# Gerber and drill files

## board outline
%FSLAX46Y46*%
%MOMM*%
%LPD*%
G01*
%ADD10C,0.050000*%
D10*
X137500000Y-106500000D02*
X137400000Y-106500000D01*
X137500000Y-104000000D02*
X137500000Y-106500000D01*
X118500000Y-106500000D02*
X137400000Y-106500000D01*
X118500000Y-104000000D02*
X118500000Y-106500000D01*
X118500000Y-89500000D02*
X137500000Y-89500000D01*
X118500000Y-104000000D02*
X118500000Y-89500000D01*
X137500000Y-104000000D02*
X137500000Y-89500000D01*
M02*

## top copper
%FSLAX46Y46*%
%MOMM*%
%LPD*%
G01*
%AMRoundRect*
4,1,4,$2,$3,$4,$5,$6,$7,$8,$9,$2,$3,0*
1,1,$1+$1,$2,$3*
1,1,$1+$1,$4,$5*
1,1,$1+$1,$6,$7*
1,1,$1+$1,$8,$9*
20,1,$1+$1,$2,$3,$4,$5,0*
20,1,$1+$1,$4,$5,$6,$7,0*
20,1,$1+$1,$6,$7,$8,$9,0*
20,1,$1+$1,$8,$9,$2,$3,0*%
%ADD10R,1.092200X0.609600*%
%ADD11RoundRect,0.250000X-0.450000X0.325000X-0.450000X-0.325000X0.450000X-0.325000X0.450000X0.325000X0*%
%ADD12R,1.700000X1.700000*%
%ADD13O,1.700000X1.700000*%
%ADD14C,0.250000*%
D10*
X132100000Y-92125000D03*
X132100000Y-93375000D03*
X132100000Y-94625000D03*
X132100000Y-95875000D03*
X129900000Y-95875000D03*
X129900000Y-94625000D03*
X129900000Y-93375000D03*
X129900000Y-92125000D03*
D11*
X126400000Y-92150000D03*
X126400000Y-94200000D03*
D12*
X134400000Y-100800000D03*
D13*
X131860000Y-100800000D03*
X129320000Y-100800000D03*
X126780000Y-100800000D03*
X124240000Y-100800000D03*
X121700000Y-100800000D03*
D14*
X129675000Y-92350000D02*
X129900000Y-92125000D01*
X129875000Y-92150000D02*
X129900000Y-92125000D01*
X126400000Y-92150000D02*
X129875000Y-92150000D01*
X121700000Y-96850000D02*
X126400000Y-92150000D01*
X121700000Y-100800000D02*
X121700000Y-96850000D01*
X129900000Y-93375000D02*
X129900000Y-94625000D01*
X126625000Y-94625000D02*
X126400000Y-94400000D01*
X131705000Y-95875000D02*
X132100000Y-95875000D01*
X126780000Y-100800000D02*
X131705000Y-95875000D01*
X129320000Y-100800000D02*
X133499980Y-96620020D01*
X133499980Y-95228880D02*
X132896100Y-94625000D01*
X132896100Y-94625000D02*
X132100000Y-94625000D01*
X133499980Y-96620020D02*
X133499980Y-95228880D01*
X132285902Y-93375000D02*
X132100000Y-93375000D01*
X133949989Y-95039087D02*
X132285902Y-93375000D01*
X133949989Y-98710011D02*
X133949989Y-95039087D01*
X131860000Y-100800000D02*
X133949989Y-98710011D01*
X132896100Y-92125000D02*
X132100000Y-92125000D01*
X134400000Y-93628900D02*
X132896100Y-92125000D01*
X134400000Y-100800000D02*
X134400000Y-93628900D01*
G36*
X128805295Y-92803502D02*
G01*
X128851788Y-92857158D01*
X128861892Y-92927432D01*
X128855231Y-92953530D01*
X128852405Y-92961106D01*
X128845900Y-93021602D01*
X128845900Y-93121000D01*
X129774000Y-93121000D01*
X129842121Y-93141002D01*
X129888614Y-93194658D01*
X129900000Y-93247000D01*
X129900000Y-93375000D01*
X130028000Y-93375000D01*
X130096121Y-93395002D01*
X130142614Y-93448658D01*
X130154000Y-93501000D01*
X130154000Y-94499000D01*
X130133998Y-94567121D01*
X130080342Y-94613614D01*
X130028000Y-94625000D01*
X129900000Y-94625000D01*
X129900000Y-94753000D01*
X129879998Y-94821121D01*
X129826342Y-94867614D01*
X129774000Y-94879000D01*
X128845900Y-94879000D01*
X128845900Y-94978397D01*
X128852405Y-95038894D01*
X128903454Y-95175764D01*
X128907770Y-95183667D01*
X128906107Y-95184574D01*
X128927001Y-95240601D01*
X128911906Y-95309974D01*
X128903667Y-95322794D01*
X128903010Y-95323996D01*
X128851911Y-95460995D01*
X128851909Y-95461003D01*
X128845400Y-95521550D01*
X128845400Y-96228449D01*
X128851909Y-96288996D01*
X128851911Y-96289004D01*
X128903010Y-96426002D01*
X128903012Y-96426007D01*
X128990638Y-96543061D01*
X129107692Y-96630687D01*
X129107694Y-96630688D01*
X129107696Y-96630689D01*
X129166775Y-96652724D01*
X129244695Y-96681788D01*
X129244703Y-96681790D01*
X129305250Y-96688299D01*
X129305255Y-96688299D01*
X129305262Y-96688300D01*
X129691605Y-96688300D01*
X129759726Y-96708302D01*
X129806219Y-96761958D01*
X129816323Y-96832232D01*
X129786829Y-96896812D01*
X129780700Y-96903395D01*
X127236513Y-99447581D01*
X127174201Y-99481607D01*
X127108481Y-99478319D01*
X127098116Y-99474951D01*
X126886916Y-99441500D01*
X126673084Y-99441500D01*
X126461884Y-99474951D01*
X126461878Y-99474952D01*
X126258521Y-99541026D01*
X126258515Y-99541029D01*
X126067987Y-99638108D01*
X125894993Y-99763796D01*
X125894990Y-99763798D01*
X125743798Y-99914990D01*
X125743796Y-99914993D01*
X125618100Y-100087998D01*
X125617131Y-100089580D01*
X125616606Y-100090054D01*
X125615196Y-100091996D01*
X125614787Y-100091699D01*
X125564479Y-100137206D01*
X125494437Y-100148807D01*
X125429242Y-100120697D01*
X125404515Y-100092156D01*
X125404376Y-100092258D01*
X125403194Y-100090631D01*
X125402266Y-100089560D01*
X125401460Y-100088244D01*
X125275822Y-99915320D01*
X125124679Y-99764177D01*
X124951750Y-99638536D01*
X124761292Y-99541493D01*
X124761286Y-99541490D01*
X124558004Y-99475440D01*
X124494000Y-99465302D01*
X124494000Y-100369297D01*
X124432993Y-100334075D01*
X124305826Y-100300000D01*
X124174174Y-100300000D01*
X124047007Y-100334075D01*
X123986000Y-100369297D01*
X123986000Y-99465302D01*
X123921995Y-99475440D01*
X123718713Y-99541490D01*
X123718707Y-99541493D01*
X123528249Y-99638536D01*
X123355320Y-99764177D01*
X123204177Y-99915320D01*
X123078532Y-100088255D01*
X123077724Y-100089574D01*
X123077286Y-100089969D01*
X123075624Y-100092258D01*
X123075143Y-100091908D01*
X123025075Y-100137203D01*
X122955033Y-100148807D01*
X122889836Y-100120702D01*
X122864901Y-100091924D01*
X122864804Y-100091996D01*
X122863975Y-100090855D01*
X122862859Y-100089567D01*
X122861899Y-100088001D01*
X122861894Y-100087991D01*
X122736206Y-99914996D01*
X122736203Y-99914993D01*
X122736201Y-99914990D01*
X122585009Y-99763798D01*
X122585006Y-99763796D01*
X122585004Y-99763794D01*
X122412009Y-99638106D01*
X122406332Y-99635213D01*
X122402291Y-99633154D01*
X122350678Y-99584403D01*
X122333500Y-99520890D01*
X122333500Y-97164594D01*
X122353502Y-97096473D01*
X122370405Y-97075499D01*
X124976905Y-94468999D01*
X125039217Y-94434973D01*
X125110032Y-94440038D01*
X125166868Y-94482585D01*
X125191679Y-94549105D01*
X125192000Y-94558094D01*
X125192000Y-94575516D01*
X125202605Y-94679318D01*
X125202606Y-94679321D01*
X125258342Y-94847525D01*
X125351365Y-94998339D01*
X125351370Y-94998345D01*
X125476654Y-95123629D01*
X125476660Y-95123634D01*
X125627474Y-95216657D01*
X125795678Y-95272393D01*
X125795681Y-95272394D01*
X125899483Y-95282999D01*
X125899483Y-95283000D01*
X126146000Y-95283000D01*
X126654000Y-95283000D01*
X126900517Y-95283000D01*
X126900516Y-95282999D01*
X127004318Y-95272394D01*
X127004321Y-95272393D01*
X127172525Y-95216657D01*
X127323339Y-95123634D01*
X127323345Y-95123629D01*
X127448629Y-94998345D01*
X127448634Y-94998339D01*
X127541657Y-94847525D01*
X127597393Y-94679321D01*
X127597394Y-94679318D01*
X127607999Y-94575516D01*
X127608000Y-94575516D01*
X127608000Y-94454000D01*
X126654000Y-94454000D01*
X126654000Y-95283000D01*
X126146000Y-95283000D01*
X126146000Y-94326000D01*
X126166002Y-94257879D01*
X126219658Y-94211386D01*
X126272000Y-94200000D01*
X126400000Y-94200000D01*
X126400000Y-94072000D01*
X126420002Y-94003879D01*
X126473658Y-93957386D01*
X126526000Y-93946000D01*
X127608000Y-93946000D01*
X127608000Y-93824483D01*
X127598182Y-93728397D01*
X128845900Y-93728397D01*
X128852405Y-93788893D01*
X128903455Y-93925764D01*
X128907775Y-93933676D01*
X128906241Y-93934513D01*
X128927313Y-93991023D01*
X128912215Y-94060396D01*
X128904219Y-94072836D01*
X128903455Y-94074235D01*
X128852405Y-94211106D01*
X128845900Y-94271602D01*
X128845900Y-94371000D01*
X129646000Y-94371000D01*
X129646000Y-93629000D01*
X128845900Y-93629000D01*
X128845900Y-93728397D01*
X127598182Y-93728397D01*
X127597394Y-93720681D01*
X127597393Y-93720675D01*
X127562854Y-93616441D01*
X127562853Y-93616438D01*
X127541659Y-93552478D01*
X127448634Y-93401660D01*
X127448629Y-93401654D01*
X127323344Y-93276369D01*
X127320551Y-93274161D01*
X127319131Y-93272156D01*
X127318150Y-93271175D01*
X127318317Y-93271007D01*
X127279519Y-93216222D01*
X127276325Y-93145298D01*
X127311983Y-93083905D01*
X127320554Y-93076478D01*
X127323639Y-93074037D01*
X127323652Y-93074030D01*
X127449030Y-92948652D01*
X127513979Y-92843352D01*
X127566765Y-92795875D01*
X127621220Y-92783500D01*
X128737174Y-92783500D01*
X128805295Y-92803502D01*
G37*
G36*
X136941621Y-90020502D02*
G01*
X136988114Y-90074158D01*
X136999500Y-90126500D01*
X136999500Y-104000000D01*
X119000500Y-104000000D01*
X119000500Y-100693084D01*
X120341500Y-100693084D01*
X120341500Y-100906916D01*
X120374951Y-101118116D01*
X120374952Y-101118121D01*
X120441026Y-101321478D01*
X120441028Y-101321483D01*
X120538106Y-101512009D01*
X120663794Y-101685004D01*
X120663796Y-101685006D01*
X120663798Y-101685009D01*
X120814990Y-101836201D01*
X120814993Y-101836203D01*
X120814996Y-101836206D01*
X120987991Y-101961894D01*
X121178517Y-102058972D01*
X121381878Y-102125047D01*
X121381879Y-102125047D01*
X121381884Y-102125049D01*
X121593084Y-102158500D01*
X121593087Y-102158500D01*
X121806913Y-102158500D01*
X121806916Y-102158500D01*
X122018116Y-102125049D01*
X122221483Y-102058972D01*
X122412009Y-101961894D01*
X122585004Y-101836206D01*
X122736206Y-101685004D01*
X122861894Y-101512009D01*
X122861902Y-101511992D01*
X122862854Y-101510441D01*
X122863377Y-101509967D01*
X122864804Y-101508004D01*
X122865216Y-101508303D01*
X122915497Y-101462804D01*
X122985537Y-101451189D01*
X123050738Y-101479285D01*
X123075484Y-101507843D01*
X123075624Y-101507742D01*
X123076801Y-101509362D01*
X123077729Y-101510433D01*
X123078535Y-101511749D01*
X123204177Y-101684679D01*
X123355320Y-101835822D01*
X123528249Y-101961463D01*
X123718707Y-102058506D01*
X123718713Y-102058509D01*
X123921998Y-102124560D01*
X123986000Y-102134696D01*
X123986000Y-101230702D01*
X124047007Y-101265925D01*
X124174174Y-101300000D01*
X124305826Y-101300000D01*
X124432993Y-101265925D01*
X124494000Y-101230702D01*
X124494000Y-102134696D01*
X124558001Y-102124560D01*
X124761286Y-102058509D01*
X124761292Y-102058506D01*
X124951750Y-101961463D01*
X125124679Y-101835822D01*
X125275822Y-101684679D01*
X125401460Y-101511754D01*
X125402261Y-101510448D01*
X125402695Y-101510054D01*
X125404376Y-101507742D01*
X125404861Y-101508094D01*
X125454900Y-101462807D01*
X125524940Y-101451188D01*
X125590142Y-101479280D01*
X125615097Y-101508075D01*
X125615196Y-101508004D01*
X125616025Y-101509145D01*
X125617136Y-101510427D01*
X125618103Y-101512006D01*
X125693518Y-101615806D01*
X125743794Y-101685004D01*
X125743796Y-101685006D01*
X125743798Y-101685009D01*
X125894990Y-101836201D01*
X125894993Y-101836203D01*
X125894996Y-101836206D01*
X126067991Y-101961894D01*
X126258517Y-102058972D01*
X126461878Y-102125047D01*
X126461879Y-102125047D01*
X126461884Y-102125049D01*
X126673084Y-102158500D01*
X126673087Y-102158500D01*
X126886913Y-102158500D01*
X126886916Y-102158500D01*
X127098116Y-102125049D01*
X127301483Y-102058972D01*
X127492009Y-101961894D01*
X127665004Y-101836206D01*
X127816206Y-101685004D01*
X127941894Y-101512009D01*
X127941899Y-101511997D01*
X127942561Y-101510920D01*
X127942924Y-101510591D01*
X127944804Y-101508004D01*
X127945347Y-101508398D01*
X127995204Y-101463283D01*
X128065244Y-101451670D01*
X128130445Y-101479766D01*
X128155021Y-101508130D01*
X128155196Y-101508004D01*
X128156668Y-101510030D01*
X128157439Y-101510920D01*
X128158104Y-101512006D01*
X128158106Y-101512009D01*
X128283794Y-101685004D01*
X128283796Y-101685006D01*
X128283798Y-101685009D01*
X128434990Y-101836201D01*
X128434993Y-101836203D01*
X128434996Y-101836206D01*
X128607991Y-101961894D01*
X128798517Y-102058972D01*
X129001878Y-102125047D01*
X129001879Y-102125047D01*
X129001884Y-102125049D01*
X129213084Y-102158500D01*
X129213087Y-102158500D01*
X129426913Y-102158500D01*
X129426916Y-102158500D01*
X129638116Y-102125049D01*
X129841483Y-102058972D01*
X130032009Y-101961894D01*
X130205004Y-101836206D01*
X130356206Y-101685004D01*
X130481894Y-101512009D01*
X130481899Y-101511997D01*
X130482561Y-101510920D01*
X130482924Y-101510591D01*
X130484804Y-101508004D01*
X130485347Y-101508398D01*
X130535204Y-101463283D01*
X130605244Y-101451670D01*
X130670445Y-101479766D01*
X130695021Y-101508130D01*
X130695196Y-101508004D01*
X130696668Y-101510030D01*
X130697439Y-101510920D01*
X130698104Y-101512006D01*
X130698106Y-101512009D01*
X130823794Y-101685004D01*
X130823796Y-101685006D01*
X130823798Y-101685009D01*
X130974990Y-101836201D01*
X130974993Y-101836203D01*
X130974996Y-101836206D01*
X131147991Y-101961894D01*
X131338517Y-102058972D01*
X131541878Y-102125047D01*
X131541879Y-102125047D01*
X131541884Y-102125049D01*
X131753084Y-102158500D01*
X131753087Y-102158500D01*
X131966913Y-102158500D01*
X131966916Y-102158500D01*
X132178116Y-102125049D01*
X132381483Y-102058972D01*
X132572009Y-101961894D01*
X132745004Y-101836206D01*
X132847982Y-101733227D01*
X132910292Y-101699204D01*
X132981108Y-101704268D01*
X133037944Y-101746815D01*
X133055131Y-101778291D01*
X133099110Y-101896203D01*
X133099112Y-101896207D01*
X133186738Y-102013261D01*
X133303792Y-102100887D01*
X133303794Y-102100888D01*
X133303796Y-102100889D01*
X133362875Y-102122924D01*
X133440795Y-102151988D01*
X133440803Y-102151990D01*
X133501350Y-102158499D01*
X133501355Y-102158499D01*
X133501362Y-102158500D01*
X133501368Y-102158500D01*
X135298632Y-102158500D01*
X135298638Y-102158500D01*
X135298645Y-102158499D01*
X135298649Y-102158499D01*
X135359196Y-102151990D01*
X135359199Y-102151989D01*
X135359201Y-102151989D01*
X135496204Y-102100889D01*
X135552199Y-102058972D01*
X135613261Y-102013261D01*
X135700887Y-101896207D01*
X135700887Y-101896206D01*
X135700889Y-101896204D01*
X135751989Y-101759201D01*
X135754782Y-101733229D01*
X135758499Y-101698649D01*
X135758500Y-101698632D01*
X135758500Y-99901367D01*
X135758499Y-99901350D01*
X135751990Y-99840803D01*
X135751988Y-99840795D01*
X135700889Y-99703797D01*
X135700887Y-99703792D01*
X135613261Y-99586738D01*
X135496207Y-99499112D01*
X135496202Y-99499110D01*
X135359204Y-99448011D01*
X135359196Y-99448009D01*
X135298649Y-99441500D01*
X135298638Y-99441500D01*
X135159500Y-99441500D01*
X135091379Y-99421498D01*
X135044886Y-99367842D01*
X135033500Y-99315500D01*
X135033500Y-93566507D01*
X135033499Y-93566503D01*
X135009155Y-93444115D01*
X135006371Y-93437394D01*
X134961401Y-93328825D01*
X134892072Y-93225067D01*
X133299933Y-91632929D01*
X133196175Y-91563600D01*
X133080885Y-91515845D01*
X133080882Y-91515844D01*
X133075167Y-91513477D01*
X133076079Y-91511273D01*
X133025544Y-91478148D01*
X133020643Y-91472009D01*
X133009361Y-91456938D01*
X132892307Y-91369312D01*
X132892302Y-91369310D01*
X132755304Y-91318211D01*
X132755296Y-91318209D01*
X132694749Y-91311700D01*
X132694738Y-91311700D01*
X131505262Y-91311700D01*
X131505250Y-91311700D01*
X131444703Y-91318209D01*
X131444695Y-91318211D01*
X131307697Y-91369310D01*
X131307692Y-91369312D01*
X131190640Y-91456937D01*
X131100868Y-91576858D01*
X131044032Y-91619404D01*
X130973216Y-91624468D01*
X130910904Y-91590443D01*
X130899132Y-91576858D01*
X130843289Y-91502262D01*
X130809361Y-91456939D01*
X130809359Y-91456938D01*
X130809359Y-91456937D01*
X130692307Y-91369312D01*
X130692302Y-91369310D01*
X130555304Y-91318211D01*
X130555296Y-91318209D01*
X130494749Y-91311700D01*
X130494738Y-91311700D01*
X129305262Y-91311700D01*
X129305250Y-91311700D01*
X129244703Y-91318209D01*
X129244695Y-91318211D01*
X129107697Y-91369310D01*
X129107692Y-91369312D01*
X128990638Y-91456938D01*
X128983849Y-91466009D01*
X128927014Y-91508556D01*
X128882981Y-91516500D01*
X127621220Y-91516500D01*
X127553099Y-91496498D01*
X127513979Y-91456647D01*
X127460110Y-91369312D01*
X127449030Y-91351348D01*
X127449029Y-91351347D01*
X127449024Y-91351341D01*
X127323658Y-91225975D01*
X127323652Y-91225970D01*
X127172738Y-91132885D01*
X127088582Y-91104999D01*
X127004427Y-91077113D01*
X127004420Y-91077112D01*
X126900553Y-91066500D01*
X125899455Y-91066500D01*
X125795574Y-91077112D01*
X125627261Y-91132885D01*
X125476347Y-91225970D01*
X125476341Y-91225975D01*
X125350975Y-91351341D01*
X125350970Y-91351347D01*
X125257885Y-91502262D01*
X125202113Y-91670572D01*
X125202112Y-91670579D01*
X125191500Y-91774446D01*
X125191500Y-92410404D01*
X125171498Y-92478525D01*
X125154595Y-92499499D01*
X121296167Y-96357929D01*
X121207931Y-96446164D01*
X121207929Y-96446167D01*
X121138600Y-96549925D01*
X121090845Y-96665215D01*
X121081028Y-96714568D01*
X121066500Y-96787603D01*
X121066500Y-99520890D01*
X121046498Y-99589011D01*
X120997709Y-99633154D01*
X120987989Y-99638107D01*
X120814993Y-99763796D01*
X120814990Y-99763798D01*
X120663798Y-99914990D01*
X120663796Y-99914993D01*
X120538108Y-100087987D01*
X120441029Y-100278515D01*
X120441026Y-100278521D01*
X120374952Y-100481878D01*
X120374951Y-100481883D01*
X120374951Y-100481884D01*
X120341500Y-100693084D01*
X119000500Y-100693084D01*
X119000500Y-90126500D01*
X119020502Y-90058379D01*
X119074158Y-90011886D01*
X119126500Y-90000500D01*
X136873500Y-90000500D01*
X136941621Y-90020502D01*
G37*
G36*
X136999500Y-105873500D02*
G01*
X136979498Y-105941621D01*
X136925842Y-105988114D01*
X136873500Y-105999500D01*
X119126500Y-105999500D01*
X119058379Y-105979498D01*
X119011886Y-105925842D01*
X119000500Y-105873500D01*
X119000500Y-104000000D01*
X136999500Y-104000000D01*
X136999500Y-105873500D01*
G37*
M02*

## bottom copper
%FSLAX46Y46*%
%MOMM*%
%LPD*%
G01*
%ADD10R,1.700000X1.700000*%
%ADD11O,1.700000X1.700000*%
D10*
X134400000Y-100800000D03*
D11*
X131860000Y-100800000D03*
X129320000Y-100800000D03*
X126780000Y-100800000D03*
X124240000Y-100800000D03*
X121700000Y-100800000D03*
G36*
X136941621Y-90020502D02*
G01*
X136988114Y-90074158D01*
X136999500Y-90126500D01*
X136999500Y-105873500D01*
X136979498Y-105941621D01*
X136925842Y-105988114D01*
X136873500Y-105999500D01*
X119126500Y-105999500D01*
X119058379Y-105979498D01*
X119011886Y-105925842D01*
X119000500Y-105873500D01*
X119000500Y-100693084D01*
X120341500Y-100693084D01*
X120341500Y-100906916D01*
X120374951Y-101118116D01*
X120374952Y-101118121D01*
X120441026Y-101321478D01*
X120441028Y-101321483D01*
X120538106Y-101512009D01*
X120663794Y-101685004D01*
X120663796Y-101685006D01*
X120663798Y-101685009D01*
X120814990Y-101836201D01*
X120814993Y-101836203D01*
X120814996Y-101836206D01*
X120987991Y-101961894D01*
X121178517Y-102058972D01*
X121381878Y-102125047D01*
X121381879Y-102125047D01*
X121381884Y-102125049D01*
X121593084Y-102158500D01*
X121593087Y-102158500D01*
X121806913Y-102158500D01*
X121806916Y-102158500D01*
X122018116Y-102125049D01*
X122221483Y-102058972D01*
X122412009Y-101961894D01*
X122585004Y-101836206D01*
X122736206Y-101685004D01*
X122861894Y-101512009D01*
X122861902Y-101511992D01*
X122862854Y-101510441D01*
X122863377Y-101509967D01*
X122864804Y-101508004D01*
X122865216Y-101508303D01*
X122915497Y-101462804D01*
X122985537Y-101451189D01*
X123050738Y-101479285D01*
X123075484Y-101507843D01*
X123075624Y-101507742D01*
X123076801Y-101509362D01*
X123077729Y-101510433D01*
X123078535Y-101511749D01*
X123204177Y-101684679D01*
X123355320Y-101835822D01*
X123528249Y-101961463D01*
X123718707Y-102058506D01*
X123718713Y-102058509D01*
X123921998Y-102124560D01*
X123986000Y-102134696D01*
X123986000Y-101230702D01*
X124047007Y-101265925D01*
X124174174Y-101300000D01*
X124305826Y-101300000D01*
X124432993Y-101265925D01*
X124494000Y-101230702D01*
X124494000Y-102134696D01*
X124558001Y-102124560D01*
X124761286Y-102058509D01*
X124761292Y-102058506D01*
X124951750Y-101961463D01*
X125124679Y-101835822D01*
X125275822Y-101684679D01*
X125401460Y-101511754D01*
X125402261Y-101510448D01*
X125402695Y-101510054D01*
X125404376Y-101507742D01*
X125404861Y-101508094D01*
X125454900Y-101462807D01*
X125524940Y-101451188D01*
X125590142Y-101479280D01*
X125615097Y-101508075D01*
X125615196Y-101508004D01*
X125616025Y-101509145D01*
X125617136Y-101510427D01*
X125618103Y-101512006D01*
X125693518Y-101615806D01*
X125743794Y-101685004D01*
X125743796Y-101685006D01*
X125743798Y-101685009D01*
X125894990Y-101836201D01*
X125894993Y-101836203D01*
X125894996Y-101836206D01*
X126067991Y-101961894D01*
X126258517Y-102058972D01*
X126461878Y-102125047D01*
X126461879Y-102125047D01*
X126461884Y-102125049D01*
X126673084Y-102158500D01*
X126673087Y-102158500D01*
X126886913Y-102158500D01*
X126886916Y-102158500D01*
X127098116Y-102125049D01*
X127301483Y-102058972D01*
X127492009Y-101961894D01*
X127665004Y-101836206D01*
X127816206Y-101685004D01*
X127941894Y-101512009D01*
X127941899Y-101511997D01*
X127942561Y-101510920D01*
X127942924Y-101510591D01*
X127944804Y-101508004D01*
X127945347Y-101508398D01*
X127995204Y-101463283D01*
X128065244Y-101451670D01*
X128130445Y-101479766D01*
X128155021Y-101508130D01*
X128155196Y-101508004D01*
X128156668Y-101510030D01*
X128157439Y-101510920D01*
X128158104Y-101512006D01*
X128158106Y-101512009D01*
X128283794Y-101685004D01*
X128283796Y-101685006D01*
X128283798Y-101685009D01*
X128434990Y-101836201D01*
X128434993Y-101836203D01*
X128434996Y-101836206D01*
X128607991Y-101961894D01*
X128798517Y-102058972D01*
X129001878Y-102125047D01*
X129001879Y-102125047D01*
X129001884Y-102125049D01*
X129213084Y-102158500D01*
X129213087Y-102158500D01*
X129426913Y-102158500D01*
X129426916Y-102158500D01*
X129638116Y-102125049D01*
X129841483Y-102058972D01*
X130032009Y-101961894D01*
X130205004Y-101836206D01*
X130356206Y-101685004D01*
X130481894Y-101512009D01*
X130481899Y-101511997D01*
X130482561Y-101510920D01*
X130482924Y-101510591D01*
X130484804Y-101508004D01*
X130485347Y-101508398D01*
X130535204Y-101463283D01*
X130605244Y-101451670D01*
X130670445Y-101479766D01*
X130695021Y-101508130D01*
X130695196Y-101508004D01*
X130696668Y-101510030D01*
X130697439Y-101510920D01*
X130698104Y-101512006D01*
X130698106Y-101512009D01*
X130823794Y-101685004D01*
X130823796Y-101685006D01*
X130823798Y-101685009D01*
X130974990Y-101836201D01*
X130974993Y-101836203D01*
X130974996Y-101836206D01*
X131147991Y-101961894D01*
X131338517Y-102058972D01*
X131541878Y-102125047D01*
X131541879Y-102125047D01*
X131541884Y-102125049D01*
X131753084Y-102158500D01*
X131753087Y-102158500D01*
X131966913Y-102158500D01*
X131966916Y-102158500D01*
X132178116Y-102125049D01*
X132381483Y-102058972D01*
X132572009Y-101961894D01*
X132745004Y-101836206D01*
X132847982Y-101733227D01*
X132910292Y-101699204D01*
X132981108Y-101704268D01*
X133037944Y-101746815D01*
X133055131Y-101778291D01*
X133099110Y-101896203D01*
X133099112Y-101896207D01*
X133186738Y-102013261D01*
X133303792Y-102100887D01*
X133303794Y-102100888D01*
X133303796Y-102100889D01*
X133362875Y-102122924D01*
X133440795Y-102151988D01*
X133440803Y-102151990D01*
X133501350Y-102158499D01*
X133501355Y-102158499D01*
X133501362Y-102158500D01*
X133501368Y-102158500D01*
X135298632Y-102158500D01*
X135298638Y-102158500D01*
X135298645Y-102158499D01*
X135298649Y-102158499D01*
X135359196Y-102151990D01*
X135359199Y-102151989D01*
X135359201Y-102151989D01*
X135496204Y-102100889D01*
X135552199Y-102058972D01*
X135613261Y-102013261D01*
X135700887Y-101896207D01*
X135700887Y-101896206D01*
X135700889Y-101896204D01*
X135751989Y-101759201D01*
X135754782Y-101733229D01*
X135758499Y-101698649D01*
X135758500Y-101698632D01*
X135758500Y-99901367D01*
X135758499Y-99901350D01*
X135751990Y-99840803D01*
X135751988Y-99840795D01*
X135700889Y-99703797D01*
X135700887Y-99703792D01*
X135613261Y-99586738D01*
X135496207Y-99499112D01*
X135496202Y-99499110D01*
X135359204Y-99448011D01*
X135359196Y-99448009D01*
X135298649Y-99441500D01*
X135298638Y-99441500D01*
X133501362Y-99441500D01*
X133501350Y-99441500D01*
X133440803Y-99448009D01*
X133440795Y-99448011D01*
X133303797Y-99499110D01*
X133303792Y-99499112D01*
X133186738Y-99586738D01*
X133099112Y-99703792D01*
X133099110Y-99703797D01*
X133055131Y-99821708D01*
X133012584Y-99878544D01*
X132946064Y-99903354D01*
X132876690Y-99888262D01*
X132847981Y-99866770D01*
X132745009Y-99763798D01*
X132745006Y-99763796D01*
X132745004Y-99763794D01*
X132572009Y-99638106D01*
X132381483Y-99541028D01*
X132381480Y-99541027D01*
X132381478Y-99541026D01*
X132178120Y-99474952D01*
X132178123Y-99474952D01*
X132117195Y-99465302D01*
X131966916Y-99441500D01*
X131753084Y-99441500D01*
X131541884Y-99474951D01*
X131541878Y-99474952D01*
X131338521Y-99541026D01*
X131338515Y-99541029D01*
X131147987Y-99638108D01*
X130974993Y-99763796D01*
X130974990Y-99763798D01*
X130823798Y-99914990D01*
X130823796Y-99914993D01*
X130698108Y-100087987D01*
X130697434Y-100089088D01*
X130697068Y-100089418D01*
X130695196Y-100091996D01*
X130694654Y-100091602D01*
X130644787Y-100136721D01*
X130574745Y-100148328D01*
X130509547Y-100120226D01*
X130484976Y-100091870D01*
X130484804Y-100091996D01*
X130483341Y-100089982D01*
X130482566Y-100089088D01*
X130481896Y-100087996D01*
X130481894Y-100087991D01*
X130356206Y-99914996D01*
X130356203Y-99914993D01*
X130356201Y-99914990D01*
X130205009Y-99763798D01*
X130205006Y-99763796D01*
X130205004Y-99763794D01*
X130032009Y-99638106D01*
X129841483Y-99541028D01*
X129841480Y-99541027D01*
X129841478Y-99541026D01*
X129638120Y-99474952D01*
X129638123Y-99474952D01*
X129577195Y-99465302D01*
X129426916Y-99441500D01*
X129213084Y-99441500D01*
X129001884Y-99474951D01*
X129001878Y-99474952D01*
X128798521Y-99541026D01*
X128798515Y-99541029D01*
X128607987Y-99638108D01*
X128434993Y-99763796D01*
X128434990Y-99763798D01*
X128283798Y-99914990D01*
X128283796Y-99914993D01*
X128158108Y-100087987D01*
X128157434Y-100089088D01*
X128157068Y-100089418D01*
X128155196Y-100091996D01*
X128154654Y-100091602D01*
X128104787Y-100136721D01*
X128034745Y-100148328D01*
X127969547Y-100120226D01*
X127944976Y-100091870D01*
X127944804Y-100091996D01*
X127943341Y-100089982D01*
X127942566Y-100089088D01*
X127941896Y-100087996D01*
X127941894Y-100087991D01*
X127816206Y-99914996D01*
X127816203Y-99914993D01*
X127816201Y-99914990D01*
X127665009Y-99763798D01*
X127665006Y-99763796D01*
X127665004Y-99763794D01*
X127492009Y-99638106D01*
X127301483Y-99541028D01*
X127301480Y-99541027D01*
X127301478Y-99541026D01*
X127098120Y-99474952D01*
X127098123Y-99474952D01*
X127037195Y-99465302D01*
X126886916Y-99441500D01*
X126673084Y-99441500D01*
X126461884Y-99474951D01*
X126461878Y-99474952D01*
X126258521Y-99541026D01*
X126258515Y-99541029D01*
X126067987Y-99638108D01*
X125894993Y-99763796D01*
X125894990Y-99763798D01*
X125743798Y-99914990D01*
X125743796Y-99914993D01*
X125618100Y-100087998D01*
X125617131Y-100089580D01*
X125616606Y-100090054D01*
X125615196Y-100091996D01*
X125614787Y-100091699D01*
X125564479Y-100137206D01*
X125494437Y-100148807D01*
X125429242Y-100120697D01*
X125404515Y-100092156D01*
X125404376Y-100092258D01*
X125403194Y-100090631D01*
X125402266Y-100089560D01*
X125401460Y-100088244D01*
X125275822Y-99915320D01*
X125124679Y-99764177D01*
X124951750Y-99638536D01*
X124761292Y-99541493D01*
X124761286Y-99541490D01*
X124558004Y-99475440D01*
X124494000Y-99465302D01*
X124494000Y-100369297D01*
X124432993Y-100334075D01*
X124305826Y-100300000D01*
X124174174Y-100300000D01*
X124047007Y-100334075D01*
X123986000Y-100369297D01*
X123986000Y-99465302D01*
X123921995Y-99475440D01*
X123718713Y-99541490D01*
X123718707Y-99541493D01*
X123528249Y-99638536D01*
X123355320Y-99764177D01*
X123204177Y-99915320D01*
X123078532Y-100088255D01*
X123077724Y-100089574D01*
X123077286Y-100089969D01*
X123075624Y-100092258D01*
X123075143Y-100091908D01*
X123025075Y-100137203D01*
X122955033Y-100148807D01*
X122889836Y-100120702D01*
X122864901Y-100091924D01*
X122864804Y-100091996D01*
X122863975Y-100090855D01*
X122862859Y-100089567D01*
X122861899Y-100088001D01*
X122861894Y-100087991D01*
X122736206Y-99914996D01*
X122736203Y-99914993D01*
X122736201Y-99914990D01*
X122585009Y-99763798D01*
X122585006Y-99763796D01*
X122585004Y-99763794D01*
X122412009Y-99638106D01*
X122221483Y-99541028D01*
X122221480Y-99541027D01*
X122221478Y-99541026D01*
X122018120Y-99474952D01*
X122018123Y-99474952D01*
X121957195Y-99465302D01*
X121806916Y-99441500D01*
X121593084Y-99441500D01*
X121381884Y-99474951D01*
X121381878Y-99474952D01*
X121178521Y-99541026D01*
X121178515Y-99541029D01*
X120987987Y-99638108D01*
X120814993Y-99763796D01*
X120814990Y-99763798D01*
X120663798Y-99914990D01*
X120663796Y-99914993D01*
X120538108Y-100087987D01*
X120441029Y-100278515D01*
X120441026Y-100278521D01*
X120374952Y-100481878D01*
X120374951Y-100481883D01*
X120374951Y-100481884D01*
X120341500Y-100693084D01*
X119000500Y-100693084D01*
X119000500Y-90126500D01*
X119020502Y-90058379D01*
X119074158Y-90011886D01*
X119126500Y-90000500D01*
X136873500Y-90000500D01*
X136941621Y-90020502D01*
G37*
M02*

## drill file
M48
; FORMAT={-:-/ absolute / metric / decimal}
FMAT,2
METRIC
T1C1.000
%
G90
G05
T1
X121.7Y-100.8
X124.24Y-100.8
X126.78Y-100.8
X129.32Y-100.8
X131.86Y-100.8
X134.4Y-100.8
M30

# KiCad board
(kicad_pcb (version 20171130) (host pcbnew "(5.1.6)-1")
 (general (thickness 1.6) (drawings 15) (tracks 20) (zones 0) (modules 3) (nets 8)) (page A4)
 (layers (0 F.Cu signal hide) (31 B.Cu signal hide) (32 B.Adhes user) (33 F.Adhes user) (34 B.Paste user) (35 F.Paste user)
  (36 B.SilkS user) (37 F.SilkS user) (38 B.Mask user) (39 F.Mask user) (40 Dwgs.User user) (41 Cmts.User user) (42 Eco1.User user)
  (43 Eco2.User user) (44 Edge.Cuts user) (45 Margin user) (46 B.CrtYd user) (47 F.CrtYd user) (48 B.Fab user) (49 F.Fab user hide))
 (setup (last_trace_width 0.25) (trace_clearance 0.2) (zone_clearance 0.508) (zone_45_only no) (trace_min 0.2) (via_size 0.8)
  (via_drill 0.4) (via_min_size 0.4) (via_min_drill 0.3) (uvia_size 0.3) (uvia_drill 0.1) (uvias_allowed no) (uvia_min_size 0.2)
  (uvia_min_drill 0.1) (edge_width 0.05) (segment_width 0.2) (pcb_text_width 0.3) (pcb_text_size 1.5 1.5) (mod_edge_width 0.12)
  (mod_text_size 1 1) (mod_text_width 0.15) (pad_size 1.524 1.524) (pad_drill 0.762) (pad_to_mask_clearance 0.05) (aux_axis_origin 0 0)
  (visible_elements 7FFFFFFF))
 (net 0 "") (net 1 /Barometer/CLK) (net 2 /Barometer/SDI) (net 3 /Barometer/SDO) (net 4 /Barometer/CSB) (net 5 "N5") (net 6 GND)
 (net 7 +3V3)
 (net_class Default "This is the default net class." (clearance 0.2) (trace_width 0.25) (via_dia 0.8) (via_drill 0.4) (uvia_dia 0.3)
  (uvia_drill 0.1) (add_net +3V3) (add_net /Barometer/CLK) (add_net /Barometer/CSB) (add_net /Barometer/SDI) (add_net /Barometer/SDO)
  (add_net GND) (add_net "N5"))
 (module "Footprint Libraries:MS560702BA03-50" (layer F.Cu) (at 131 94)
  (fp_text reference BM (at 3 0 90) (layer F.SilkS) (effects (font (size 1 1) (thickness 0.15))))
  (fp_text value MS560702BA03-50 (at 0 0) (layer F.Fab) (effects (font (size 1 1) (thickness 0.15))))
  (pad 8 smd rect (at 1.1 -1.875) (size 1.0922 0.6096) (layers F.Cu F.Paste F.Mask) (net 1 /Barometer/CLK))
  (pad 7 smd rect (at 1.1 -0.625) (size 1.0922 0.6096) (layers F.Cu F.Paste F.Mask) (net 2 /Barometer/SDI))
  (pad 6 smd rect (at 1.1 0.625) (size 1.0922 0.6096) (layers F.Cu F.Paste F.Mask) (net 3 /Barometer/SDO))
  (pad 5 smd rect (at 1.1 1.875) (size 1.0922 0.6096) (layers F.Cu F.Paste F.Mask) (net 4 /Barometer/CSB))
  (pad 4 smd rect (at -1.1 1.875) (size 1.0922 0.6096) (layers F.Cu F.Paste F.Mask) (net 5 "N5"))
  (pad 3 smd rect (at -1.1 0.625) (size 1.0922 0.6096) (layers F.Cu F.Paste F.Mask) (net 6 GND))
  (pad 2 smd rect (at -1.1 -0.625) (size 1.0922 0.6096) (layers F.Cu F.Paste F.Mask) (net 6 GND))
  (pad 1 smd rect (at -1.1 -1.875) (size 1.0922 0.6096) (layers F.Cu F.Paste F.Mask) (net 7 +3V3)))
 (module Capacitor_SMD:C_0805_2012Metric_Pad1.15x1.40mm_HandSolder (layer F.Cu) (at 126.4 93.175 270)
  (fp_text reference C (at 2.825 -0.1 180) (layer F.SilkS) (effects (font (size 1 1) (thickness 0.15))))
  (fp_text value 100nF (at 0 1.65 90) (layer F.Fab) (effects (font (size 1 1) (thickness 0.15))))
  (pad 1 smd roundrect (at -1.025 0 270) (size 1.15 1.4) (layers F.Cu F.Paste F.Mask) (roundrect_rratio 0.217391) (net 7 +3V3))
  (pad 2 smd roundrect (at 1.025 0 270) (size 1.15 1.4) (layers F.Cu F.Paste F.Mask) (roundrect_rratio 0.217391) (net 6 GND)))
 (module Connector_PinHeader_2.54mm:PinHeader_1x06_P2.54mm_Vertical (layer F.Cu) (at 134.4 100.8 270)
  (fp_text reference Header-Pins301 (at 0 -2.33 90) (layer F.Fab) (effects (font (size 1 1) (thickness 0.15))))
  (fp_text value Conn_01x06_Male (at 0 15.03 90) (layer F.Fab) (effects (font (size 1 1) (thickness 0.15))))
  (pad 1 thru_hole rect (at 0 0 270) (size 1.7 1.7) (drill 1) (layers *.Cu *.Mask) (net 1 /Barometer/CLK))
  (pad 2 thru_hole oval (at 0 2.54 270) (size 1.7 1.7) (drill 1) (layers *.Cu *.Mask) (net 2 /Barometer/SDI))
  (pad 3 thru_hole oval (at 0 5.08 270) (size 1.7 1.7) (drill 1) (layers *.Cu *.Mask) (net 3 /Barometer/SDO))
  (pad 4 thru_hole oval (at 0 7.62 270) (size 1.7 1.7) (drill 1) (layers *.Cu *.Mask) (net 4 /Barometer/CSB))
  (pad 5 thru_hole oval (at 0 10.16 270) (size 1.7 1.7) (drill 1) (layers *.Cu *.Mask) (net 6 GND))
  (pad 6 thru_hole oval (at 0 12.7 270) (size 1.7 1.7) (drill 1) (layers *.Cu *.Mask) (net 7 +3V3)))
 (gr_line (start 137.5 106.5) (end 137.4 106.5) (layer Edge.Cuts) (width 0.05))
 (gr_line (start 137.5 104) (end 137.5 106.5) (layer Edge.Cuts) (width 0.05))
 (gr_line (start 118.5 106.5) (end 137.4 106.5) (layer Edge.Cuts) (width 0.05))
 (gr_line (start 118.5 104) (end 118.5 106.5) (layer Edge.Cuts) (width 0.05))
 (gr_line (start 118.5 89.5) (end 137.5 89.5) (layer Edge.Cuts) (width 0.05))
 (gr_line (start 118.5 104) (end 118.5 89.5) (layer Edge.Cuts) (width 0.05))
 (gr_line (start 137.5 104) (end 137.5 89.5) (layer Edge.Cuts) (width 0.05))
 (segment (start 129.675 92.35) (end 129.9 92.125) (width 0.25) (layer F.Cu) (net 7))
 (segment (start 129.875 92.15) (end 129.9 92.125) (width 0.25) (layer F.Cu) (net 7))
 (segment (start 126.4 92.15) (end 129.875 92.15) (width 0.25) (layer F.Cu) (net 7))
 (segment (start 121.7 96.85) (end 126.4 92.15) (width 0.25) (layer F.Cu) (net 7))
 (segment (start 121.7 100.8) (end 121.7 96.85) (width 0.25) (layer F.Cu) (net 7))
 (segment (start 129.9 93.375) (end 129.9 94.625) (width 0.25) (layer F.Cu) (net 6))
 (segment (start 126.625 94.625) (end 126.4 94.4) (width 0.25) (layer F.Cu) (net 6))
 (segment (start 131.705 95.875) (end 132.1 95.875) (width 0.25) (layer F.Cu) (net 4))
 (segment (start 126.78 100.8) (end 131.705 95.875) (width 0.25) (layer F.Cu) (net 4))
 (segment (start 129.32 100.8) (end 133.49998 96.62002) (width 0.25) (layer F.Cu) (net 3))
 (segment (start 133.49998 95.22888) (end 132.8961 94.625) (width 0.25) (layer F.Cu) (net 3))
 (segment (start 132.8961 94.625) (end 132.1 94.625) (width 0.25) (layer F.Cu) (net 3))
 (segment (start 133.49998 96.62002) (end 133.49998 95.22888) (width 0.25) (layer F.Cu) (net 3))
 (segment (start 132.285902 93.375) (end 132.1 93.375) (width 0.25) (layer F.Cu) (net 2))
 (segment (start 133.949989 95.039087) (end 132.285902 93.375) (width 0.25) (layer F.Cu) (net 2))
 (segment (start 133.949989 98.710011) (end 133.949989 95.039087) (width 0.25) (layer F.Cu) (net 2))
 (segment (start 131.86 100.8) (end 133.949989 98.710011) (width 0.25) (layer F.Cu) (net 2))
 (segment (start 132.8961 92.125) (end 132.1 92.125) (width 0.25) (layer F.Cu) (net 1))
 (segment (start 134.4 93.6289) (end 132.8961 92.125) (width 0.25) (layer F.Cu) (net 1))
 (segment (start 134.4 100.8) (end 134.4 93.6289) (width 0.25) (layer F.Cu) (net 1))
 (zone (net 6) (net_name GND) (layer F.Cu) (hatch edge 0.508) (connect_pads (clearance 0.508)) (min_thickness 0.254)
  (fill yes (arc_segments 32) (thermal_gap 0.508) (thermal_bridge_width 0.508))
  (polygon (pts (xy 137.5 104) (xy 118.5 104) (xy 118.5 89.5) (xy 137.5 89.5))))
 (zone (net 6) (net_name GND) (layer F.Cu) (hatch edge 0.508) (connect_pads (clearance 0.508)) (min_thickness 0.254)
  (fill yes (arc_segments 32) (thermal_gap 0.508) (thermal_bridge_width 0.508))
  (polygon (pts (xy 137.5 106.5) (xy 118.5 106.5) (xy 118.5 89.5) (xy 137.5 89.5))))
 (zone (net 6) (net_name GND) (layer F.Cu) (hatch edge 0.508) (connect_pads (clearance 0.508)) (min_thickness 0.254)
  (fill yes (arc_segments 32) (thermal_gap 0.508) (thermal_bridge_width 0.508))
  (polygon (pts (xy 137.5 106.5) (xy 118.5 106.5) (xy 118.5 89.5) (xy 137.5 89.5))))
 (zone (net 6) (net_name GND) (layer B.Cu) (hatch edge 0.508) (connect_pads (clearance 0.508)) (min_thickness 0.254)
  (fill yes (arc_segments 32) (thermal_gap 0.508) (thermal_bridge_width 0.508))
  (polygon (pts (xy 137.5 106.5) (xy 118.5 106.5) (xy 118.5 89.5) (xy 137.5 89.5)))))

